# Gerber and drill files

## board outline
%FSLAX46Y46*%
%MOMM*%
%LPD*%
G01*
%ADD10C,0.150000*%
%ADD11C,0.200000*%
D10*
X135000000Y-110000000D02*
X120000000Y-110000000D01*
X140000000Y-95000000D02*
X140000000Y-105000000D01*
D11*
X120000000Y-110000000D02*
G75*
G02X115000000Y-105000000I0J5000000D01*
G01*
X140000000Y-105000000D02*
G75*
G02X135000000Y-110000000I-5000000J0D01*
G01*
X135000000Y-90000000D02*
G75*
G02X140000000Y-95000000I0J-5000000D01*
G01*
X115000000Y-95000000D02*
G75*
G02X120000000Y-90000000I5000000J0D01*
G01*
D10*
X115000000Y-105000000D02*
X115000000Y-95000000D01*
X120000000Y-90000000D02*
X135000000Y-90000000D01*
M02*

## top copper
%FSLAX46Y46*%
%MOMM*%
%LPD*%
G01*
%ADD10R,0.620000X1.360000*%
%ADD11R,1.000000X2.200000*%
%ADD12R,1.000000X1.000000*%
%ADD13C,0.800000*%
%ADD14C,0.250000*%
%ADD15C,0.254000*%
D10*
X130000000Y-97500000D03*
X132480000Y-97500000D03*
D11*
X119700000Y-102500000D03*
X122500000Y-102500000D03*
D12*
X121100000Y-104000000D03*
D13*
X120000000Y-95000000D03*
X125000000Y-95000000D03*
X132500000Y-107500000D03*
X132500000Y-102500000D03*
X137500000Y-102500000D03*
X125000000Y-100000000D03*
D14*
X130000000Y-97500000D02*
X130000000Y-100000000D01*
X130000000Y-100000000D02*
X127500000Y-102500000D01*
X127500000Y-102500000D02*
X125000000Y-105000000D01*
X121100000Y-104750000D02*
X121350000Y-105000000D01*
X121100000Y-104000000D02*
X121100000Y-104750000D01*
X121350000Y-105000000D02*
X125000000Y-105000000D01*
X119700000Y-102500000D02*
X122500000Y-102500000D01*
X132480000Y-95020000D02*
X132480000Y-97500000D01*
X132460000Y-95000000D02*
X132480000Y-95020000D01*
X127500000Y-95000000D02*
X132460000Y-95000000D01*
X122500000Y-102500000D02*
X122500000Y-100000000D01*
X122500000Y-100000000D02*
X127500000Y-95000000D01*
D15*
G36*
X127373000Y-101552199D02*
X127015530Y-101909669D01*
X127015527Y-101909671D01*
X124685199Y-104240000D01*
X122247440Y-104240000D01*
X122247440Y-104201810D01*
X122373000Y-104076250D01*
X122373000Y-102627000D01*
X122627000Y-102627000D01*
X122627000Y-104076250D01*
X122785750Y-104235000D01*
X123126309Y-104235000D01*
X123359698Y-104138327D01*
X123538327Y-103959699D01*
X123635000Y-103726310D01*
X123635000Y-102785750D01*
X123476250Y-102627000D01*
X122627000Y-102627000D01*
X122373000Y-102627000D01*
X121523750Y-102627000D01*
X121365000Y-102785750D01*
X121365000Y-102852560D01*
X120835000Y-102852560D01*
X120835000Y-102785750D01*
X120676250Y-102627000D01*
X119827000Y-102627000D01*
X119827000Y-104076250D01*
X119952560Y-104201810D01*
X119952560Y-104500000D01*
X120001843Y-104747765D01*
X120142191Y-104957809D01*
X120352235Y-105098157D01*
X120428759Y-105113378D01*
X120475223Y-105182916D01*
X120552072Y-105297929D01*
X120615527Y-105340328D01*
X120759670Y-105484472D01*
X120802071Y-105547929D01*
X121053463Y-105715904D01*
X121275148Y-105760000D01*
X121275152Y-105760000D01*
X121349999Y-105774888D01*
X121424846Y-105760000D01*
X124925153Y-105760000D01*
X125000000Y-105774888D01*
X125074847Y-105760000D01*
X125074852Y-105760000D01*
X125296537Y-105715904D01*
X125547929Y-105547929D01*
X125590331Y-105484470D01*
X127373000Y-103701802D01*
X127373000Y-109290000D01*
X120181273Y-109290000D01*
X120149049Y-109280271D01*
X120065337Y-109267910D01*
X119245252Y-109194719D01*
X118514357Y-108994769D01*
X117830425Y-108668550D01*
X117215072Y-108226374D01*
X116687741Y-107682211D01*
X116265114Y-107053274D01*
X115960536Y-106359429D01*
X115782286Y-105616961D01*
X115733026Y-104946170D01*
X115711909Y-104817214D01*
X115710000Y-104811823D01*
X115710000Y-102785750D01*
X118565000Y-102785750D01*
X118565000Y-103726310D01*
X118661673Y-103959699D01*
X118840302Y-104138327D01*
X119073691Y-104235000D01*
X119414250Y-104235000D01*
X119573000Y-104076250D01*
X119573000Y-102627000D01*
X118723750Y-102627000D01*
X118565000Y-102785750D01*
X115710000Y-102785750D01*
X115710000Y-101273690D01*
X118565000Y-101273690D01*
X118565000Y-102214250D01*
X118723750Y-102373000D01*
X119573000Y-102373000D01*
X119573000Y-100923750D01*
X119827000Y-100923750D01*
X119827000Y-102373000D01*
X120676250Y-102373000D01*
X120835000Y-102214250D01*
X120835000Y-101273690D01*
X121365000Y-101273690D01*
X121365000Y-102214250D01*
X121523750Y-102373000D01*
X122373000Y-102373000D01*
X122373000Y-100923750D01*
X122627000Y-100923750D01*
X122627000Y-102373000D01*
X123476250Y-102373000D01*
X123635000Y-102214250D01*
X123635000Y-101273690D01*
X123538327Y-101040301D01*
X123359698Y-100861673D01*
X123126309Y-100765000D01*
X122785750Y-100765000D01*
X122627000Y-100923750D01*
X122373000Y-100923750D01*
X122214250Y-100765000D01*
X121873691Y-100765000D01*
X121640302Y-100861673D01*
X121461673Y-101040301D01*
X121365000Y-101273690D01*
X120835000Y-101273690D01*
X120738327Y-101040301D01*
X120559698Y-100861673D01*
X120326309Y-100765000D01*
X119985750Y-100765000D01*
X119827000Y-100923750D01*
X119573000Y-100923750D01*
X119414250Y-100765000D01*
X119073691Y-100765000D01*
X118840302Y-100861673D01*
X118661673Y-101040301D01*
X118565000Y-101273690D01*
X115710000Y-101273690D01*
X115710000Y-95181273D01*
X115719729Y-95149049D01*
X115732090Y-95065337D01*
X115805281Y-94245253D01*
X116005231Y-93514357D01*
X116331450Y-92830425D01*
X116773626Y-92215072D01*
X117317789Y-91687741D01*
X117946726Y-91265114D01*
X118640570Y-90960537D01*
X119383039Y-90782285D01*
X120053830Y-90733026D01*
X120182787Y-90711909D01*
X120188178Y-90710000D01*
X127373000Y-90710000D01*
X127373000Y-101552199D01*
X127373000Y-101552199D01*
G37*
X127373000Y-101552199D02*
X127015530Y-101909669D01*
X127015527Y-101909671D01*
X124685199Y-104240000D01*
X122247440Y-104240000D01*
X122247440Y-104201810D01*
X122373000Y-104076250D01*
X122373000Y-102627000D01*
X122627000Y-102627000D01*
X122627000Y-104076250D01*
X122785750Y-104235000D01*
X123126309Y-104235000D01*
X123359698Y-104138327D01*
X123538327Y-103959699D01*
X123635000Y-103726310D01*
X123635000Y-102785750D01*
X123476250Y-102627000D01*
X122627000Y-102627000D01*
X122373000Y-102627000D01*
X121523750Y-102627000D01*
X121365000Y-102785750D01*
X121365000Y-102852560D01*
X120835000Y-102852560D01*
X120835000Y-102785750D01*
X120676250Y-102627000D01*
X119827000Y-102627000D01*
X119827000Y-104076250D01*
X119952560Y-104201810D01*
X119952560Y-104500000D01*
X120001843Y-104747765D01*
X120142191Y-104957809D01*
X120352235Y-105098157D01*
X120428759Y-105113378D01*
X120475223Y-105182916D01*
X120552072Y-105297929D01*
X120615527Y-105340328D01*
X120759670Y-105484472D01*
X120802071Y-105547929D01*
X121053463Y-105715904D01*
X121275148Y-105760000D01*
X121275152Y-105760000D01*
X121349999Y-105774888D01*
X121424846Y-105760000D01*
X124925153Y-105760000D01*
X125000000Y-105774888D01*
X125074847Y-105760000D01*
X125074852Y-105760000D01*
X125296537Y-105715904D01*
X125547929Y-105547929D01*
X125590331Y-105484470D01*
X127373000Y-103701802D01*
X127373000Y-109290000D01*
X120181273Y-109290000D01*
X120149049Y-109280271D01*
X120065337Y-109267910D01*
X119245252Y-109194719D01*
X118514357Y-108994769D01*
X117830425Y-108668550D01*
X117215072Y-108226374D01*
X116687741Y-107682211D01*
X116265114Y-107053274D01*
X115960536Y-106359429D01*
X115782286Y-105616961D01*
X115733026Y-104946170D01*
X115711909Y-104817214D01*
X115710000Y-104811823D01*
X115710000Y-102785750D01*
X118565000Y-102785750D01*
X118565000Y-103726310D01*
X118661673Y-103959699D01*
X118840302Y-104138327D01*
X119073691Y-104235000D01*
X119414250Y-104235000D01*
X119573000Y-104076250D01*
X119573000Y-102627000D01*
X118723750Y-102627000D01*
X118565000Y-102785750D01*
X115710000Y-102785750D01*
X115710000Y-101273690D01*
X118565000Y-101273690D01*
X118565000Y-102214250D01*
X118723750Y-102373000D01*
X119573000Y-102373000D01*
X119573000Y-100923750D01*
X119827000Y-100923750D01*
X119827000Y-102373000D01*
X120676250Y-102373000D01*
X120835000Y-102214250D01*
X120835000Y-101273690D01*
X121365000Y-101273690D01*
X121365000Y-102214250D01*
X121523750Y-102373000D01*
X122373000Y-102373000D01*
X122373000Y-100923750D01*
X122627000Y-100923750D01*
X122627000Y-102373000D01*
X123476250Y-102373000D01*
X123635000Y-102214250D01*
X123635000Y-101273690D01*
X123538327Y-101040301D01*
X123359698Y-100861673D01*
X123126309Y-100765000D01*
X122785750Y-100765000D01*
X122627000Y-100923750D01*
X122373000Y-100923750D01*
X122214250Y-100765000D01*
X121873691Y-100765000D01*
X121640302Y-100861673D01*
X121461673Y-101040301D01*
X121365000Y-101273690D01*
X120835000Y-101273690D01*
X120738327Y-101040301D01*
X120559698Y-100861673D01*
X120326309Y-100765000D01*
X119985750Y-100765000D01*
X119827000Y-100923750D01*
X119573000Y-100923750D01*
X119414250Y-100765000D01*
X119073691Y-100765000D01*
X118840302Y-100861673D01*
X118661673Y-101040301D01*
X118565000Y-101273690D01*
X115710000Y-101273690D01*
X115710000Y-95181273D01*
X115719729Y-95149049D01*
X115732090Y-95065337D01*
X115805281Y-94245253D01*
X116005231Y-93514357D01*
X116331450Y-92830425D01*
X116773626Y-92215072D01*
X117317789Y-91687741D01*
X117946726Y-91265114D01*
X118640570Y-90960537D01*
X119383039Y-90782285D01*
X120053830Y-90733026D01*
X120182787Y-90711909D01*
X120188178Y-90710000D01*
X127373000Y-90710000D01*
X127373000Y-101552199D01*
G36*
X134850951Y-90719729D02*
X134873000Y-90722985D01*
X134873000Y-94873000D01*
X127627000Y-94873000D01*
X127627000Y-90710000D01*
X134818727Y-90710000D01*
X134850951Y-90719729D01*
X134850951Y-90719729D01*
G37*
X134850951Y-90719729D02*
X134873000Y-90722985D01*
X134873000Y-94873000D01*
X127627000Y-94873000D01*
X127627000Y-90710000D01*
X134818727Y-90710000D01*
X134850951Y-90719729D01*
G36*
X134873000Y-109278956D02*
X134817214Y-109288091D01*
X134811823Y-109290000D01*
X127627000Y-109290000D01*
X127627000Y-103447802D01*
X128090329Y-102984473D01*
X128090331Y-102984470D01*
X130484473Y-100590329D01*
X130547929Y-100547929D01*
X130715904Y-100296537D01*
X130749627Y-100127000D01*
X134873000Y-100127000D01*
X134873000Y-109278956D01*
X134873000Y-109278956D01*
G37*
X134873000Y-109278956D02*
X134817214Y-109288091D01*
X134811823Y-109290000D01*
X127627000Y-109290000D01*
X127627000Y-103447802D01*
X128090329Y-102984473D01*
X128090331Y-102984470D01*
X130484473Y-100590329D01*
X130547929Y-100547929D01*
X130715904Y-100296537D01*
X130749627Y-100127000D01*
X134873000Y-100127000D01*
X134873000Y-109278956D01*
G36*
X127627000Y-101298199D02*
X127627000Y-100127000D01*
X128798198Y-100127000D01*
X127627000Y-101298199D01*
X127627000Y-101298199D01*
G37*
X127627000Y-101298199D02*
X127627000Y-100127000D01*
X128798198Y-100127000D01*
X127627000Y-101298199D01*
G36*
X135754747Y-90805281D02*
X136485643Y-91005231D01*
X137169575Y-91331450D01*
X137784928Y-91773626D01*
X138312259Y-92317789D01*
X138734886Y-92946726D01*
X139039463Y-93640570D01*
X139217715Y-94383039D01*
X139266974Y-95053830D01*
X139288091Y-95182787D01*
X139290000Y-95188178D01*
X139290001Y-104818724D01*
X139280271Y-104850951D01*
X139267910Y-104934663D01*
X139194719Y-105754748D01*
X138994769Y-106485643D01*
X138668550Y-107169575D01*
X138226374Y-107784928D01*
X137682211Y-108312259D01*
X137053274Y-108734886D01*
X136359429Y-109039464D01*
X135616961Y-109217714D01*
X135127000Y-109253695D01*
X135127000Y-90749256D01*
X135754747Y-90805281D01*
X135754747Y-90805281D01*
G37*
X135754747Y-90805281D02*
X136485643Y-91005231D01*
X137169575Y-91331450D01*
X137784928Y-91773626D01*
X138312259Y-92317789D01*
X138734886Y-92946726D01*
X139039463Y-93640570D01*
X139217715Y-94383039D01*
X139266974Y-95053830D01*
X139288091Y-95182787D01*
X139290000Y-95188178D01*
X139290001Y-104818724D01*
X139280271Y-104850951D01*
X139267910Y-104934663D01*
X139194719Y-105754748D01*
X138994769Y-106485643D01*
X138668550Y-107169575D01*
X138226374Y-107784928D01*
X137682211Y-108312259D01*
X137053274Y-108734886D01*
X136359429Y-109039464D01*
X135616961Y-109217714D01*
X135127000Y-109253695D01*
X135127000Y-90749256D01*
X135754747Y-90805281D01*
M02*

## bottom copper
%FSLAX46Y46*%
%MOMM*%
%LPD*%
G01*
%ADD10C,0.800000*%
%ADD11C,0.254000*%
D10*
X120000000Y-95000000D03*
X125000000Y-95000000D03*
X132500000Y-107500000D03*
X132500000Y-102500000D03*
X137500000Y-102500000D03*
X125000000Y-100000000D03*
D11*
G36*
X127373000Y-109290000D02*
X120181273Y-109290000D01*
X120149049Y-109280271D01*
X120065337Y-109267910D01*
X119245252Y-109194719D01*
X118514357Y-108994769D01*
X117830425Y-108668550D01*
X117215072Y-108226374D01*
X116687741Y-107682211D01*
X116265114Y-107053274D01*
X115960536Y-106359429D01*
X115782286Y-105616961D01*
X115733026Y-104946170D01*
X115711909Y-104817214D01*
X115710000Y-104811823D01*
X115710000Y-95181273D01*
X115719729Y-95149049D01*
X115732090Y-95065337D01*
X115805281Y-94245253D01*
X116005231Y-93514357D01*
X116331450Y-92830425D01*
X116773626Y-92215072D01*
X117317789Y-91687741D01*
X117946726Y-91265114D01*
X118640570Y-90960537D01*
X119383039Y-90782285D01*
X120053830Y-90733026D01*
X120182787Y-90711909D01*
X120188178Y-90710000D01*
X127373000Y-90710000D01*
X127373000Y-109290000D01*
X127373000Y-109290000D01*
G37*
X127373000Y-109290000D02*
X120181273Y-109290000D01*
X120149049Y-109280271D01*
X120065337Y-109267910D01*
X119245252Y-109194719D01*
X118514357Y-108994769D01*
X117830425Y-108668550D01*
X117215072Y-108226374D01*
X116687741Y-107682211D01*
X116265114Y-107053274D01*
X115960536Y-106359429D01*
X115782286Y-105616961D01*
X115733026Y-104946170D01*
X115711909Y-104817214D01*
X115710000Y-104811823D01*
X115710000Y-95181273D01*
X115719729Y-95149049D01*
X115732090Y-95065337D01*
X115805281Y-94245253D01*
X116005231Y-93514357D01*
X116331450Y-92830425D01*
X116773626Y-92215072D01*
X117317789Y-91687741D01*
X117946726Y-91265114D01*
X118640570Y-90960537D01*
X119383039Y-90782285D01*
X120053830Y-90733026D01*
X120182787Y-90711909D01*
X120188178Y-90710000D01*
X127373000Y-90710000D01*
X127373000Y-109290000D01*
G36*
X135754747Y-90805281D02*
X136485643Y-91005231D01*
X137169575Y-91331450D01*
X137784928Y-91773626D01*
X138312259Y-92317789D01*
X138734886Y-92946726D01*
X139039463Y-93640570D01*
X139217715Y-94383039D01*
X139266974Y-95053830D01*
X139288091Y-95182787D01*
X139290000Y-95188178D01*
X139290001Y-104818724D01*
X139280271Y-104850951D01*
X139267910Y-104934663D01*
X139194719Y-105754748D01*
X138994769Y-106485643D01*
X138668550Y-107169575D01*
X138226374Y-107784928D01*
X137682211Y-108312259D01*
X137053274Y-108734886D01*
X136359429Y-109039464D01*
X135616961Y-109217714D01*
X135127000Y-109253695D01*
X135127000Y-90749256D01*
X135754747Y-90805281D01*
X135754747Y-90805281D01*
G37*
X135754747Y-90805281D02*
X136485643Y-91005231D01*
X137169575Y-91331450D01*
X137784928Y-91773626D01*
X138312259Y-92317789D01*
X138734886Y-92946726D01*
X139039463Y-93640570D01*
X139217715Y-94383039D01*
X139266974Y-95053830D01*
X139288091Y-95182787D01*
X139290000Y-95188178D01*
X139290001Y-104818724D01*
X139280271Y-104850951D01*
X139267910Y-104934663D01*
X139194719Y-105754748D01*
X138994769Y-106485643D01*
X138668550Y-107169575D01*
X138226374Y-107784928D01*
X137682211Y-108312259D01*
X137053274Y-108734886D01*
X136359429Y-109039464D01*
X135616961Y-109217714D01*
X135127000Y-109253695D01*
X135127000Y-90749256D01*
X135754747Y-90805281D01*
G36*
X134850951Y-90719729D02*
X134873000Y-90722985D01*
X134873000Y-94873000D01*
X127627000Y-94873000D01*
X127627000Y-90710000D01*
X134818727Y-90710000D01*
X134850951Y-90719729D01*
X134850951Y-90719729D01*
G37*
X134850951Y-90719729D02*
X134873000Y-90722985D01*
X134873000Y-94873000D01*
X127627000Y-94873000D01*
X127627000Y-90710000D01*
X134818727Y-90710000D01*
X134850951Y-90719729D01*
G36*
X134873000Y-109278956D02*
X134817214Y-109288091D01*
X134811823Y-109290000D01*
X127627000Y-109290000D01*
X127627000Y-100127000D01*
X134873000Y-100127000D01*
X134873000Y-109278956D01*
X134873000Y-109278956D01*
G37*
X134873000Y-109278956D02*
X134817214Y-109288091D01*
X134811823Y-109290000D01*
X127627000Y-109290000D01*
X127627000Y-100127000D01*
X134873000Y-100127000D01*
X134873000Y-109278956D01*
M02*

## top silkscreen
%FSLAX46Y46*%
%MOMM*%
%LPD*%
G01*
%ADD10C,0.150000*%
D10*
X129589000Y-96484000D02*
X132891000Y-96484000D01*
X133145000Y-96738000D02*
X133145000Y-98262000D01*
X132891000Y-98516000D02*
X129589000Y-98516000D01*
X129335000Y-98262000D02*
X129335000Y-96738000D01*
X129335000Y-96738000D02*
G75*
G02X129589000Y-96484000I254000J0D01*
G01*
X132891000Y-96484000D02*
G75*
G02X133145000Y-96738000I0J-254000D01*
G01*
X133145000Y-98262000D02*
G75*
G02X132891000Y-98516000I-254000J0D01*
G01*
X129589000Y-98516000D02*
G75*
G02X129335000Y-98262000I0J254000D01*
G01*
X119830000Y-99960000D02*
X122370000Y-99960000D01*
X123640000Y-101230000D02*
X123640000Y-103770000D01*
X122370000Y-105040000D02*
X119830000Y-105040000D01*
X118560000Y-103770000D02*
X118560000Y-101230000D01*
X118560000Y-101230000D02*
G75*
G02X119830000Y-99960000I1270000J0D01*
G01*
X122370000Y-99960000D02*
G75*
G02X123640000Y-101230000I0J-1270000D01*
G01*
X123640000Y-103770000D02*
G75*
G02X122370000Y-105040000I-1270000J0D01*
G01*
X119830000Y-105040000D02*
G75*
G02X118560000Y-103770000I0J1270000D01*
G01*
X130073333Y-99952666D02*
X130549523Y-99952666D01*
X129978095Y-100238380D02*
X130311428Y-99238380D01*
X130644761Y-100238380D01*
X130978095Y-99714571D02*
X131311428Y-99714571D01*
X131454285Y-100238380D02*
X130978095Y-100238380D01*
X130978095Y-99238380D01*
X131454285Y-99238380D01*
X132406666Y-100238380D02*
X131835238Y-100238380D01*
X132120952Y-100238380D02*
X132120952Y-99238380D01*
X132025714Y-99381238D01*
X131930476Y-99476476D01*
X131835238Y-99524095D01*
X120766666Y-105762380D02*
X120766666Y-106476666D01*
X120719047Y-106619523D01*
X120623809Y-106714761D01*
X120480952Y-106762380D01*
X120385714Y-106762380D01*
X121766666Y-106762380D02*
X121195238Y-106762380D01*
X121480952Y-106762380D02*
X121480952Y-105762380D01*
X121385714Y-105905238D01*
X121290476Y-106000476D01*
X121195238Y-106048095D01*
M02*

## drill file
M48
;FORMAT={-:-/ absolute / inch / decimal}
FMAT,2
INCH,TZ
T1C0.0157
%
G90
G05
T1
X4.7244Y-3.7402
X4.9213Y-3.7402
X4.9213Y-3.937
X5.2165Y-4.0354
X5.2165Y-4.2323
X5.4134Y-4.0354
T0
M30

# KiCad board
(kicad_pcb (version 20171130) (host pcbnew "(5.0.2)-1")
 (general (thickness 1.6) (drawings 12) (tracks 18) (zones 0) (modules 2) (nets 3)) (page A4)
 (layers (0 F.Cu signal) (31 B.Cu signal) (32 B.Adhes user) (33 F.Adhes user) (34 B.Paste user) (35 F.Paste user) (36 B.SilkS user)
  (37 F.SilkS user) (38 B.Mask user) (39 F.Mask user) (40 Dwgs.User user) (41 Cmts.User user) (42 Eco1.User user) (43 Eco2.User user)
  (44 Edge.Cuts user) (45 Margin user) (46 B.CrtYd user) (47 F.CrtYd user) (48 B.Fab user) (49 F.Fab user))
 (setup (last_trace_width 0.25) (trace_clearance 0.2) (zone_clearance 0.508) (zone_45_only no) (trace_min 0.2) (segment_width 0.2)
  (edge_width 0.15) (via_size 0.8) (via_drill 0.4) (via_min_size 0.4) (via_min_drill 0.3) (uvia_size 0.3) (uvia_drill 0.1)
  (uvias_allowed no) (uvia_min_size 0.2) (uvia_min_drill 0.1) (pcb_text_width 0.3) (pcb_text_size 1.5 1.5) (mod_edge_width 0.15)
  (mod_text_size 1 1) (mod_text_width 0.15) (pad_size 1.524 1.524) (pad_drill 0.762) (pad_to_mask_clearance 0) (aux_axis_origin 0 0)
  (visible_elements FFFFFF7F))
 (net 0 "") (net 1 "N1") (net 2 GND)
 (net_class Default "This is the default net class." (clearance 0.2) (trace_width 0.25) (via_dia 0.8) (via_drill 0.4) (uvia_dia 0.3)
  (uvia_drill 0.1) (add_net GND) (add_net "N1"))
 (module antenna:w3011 (layer F.Cu) (at 131.24 97.5)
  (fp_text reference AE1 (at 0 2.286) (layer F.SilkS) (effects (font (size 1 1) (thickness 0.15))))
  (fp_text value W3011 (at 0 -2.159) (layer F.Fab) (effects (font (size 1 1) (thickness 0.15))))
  (fp_line (start -1.651 -1.016) (end 1.651 -1.016) (layer F.SilkS) (width 0.15))
  (fp_line (start 1.905 -0.762) (end 1.905 0.762) (layer F.SilkS) (width 0.15))
  (fp_line (start 1.651 1.016) (end -1.651 1.016) (layer F.SilkS) (width 0.15))
  (fp_line (start -1.905 0.762) (end -1.905 -0.762) (layer F.SilkS) (width 0.15))
  (fp_arc (start -1.651 -0.762) (end -1.651 -1.016) (angle -90) (layer F.SilkS) (width 0.15))
  (fp_arc (start 1.651 -0.762) (end 1.905 -0.762) (angle -90) (layer F.SilkS) (width 0.15))
  (fp_arc (start 1.651 0.762) (end 1.651 1.016) (angle -90) (layer F.SilkS) (width 0.15))
  (fp_arc (start -1.651 0.762) (end -1.905 0.762) (angle -90) (layer F.SilkS) (width 0.15))
  (pad 1 smd rect (at -1.24 0) (size 0.62 1.36) (layers F.Cu F.Paste F.Mask) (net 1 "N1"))
  (pad 2 smd rect (at 1.24 0) (size 0.62 1.36) (layers F.Cu F.Paste F.Mask) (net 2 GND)))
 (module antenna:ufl (layer F.Cu) (at 121.1 102.5)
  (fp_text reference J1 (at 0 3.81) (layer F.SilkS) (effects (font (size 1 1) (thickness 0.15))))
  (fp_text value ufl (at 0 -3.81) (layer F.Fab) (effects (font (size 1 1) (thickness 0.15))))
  (fp_line (start -1.27 -2.54) (end 1.27 -2.54) (layer F.SilkS) (width 0.15))
  (fp_line (start 2.54 -1.27) (end 2.54 1.27) (layer F.SilkS) (width 0.15))
  (fp_line (start 1.27 2.54) (end -1.27 2.54) (layer F.SilkS) (width 0.15))
  (fp_line (start -2.54 1.27) (end -2.54 -1.27) (layer F.SilkS) (width 0.15))
  (fp_arc (start -1.27 -1.27) (end -1.27 -2.54) (angle -90) (layer F.SilkS) (width 0.15))
  (fp_arc (start 1.27 -1.27) (end 2.54 -1.27) (angle -90) (layer F.SilkS) (width 0.15))
  (fp_arc (start 1.27 1.27) (end 1.27 2.54) (angle -90) (layer F.SilkS) (width 0.15))
  (fp_arc (start -1.27 1.27) (end -2.54 1.27) (angle -90) (layer F.SilkS) (width 0.15))
  (pad 1 smd rect (at -1.4 0) (size 1 2.2) (layers F.Cu F.Paste F.Mask) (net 2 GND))
  (pad 1 smd rect (at 1.4 0) (size 1 2.2) (layers F.Cu F.Paste F.Mask) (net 2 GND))
  (pad 2 smd rect (at 0 1.5) (size 1 1) (layers F.Cu F.Paste F.Mask) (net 1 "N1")))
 (gr_line (start 135 110) (end 120 110) (layer Edge.Cuts) (width 0.15))
 (gr_line (start 140 95) (end 140 105) (layer Edge.Cuts) (width 0.15))
 (gr_arc (start 120 105) (end 115 105) (angle -90) (layer Edge.Cuts) (width 0.2))
 (gr_arc (start 135 105) (end 135 110) (angle -90) (layer Edge.Cuts) (width 0.2))
 (gr_arc (start 135 95) (end 140 95) (angle -90) (layer Edge.Cuts) (width 0.2))
 (gr_arc (start 120 95) (end 120 90) (angle -90) (layer Edge.Cuts) (width 0.2))
 (gr_line (start 115 105) (end 115 95) (layer Edge.Cuts) (width 0.15))
 (gr_line (start 120 90) (end 135 90) (layer Edge.Cuts) (width 0.15))
 (segment (start 130 97.5) (end 130 100) (width 0.25) (layer F.Cu) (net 1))
 (segment (start 130 100) (end 127.5 102.5) (width 0.25) (layer F.Cu) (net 1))
 (segment (start 127.5 102.5) (end 125 105) (width 0.25) (layer F.Cu) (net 1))
 (segment (start 121.1 104.75) (end 121.35 105) (width 0.25) (layer F.Cu) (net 1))
 (segment (start 121.1 104) (end 121.1 104.75) (width 0.25) (layer F.Cu) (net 1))
 (segment (start 121.35 105) (end 125 105) (width 0.25) (layer F.Cu) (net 1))
 (segment (start 119.7 102.5) (end 122.5 102.5) (width 0.25) (layer F.Cu) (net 2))
 (segment (start 132.48 95.02) (end 132.48 97.5) (width 0.25) (layer F.Cu) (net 2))
 (segment (start 132.46 95) (end 132.48 95.02) (width 0.25) (layer F.Cu) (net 2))
 (segment (start 127.5 95) (end 132.46 95) (width 0.25) (layer F.Cu) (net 2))
 (segment (start 122.5 102.5) (end 122.5 100) (width 0.25) (layer F.Cu) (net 2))
 (segment (start 122.5 100) (end 127.5 95) (width 0.25) (layer F.Cu) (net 2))
 (via (at 120 95) (size 0.8) (drill 0.4) (layers F.Cu B.Cu) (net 2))
 (via (at 125 95) (size 0.8) (drill 0.4) (layers F.Cu B.Cu) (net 2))
 (via (at 132.5 107.5) (size 0.8) (drill 0.4) (layers F.Cu B.Cu) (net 2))
 (via (at 132.5 102.5) (size 0.8) (drill 0.4) (layers F.Cu B.Cu) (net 2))
 (via (at 137.5 102.5) (size 0.8) (drill 0.4) (layers F.Cu B.Cu) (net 2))
 (via (at 125 100) (size 0.8) (drill 0.4) (layers F.Cu B.Cu) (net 2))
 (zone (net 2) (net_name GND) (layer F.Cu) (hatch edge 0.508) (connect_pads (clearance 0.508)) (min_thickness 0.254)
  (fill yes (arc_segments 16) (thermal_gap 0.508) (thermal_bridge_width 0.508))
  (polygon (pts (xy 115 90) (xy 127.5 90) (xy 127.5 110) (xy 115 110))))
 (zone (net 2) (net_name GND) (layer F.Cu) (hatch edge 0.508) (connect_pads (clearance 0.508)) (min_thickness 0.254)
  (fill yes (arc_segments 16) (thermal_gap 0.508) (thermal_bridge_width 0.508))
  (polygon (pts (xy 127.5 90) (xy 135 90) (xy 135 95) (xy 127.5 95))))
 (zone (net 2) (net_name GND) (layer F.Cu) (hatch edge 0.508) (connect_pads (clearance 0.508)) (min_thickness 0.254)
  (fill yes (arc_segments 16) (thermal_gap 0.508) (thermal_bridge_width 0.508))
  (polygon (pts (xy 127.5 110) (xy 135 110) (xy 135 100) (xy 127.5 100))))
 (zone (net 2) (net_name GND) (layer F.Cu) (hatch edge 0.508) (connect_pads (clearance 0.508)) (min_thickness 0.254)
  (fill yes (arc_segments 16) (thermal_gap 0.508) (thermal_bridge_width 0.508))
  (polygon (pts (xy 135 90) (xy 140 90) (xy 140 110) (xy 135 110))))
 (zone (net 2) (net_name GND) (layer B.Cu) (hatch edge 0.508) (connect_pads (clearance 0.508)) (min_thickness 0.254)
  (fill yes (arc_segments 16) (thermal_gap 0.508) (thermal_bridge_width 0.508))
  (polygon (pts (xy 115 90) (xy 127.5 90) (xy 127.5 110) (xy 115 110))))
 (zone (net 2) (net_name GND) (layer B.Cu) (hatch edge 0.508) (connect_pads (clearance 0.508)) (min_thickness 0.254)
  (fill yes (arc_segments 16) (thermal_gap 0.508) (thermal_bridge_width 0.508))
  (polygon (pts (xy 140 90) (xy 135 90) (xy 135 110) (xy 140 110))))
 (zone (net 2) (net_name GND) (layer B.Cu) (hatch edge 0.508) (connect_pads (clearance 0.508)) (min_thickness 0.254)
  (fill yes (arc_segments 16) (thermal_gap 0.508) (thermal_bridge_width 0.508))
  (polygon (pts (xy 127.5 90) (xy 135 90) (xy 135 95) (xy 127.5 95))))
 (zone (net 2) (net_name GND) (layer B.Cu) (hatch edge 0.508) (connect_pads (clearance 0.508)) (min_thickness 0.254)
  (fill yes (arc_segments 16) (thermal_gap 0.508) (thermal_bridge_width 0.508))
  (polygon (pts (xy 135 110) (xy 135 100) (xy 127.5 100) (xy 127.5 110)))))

